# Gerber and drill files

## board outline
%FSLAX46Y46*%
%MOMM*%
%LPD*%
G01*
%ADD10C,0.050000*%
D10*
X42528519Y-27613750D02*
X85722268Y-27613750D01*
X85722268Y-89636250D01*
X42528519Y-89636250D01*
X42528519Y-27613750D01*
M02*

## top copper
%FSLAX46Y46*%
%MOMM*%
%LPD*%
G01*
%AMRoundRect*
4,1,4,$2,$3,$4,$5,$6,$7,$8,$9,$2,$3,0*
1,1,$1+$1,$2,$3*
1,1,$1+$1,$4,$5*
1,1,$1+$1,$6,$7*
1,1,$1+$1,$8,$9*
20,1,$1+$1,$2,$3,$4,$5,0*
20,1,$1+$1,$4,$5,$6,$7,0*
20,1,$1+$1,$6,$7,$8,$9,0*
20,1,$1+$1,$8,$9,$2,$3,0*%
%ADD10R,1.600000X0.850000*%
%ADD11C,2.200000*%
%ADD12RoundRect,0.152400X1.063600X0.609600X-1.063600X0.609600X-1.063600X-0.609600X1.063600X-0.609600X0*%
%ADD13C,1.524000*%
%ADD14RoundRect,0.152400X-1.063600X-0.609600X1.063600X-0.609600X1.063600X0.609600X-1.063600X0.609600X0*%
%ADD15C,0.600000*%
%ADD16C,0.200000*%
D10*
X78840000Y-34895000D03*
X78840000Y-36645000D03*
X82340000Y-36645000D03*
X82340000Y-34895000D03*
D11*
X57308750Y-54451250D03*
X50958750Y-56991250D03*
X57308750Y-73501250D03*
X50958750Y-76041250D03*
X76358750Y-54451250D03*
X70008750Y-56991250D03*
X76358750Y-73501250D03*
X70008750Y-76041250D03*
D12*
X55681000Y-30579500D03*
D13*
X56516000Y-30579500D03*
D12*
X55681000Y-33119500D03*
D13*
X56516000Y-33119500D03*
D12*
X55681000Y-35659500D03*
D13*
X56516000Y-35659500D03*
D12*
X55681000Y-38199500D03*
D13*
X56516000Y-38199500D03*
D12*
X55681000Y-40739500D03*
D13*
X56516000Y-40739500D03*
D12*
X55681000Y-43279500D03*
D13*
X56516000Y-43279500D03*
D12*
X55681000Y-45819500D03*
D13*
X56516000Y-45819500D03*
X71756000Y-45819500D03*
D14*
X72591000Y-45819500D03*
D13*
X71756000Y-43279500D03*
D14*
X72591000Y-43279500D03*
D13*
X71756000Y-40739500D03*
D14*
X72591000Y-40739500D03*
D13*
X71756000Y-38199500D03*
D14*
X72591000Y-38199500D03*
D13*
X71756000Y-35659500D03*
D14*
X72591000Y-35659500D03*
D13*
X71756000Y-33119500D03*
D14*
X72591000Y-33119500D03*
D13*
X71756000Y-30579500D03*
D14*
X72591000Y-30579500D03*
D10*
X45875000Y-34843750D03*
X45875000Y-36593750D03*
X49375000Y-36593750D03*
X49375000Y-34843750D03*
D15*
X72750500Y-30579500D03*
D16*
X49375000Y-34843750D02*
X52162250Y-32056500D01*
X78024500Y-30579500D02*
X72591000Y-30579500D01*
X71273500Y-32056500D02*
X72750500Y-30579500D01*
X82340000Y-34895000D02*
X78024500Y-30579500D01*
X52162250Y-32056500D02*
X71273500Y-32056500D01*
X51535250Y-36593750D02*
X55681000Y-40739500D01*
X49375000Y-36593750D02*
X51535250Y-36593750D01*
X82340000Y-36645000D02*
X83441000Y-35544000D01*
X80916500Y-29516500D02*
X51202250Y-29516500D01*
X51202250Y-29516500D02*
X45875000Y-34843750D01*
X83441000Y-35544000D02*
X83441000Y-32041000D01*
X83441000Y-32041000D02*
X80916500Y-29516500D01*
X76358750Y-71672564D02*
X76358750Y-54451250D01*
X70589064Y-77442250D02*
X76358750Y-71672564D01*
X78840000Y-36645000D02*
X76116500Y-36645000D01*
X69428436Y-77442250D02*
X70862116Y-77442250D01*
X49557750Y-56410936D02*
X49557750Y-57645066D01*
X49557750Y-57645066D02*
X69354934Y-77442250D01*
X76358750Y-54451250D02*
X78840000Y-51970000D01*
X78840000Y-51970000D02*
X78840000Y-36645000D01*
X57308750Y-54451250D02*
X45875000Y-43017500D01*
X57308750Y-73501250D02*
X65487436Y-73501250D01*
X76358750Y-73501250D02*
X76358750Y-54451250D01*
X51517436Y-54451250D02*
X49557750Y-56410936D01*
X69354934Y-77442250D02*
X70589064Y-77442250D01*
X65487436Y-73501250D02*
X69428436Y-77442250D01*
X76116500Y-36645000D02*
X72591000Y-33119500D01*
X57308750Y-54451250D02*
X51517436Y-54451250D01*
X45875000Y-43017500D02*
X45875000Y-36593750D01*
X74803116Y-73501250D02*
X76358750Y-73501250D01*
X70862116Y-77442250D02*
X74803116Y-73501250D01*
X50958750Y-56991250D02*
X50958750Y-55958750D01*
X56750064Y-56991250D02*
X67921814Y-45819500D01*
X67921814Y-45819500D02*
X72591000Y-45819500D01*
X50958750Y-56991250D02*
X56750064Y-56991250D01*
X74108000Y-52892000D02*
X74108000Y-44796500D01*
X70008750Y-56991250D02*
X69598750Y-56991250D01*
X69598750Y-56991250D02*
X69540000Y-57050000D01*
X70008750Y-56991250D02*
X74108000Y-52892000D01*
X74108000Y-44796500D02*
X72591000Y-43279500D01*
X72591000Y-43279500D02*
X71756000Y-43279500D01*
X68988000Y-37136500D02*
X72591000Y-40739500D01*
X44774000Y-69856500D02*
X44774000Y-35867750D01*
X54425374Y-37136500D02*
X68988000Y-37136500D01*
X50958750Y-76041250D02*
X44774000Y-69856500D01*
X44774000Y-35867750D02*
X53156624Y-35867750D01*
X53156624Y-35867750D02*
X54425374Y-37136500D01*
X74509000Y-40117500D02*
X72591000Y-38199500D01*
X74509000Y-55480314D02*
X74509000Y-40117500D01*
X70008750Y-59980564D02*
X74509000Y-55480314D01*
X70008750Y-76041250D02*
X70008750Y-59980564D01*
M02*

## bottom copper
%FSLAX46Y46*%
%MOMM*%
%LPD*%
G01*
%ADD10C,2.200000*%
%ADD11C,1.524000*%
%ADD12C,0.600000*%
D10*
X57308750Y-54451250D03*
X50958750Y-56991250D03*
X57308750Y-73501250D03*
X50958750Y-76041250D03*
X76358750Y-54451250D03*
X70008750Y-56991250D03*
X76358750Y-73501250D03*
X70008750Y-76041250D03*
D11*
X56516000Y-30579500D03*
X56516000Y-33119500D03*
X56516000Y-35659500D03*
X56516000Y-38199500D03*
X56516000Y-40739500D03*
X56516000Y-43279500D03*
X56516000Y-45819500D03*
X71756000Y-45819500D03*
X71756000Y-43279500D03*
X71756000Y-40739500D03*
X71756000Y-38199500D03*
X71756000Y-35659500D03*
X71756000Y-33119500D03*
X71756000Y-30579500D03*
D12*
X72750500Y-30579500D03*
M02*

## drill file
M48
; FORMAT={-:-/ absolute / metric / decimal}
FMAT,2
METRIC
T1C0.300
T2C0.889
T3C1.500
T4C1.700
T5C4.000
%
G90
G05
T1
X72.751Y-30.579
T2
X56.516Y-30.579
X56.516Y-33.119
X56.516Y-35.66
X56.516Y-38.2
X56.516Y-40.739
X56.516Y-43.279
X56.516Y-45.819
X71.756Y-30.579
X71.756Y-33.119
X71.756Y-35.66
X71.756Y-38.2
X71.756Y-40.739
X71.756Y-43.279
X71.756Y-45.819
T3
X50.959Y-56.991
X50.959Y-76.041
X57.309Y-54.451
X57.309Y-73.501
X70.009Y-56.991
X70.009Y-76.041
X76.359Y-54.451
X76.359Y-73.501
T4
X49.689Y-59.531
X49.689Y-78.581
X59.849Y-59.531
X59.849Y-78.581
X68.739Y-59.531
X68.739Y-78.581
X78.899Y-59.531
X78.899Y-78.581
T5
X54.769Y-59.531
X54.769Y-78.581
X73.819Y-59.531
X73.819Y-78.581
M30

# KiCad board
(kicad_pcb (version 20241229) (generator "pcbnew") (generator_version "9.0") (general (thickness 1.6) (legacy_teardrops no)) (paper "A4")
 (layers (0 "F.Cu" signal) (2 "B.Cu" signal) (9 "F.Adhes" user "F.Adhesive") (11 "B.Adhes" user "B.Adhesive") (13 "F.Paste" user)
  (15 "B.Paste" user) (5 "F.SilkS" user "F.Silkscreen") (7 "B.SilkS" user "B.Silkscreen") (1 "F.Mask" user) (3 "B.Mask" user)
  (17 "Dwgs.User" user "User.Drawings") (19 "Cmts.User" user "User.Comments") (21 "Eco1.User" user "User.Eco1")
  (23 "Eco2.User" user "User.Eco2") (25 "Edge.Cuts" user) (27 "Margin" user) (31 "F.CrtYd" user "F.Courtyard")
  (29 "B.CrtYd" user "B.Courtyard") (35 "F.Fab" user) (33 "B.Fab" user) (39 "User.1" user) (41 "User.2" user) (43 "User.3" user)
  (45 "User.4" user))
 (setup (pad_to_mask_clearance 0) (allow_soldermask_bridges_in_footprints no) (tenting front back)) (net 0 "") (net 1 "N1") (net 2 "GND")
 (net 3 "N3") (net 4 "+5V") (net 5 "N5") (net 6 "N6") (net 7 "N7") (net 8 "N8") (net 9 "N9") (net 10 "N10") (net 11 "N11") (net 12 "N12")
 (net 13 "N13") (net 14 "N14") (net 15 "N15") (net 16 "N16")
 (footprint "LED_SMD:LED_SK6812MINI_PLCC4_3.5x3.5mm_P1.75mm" (layer "F.Cu") (at 80.59 35.77)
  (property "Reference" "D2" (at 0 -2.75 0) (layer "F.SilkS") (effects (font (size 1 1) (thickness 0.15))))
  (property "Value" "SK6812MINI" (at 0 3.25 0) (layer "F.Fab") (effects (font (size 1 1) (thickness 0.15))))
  (pad "1" smd rect (at -1.75 -0.875) (size 1.6 0.85) (layers "F.Cu" "F.Mask" "F.Paste") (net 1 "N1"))
  (pad "2" smd rect (at -1.75 0.875) (size 1.6 0.85) (layers "F.Cu" "F.Mask" "F.Paste") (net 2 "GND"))
  (pad "3" smd rect (at 1.75 0.875) (size 1.6 0.85) (layers "F.Cu" "F.Mask" "F.Paste") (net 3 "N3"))
  (pad "4" smd rect (at 1.75 -0.875) (size 1.6 0.85) (layers "F.Cu" "F.Mask" "F.Paste") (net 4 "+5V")))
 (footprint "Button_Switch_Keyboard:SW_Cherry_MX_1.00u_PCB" (layer "F.Cu") (at 57.30875 54.45125)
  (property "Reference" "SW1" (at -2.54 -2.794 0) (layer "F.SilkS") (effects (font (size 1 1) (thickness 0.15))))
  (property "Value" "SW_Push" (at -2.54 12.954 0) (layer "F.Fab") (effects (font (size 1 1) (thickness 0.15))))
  (pad "" np_thru_hole circle (at -7.62 5.08) (size 1.7 1.7) (drill 1.7) (layers "*.Cu" "*.Mask"))
  (pad "" np_thru_hole circle (at -2.54 5.08) (size 4 4) (drill 4) (layers "*.Cu" "*.Mask"))
  (pad "" np_thru_hole circle (at 2.54 5.08) (size 1.7 1.7) (drill 1.7) (layers "*.Cu" "*.Mask"))
  (pad "1" thru_hole circle (at 0 0) (size 2.2 2.2) (drill 1.5) (layers "*.Cu" "*.Mask") (remove_unused_layers no) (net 2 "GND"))
  (pad "2" thru_hole circle (at -6.35 2.54) (size 2.2 2.2) (drill 1.5) (layers "*.Cu" "*.Mask") (remove_unused_layers no) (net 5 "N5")))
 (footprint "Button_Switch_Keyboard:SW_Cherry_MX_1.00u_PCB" (layer "F.Cu") (at 57.30875 73.50125)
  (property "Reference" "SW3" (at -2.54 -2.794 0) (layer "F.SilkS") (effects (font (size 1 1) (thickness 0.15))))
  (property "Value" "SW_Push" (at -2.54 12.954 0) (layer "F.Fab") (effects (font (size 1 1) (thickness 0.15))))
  (pad "" np_thru_hole circle (at -7.62 5.08) (size 1.7 1.7) (drill 1.7) (layers "*.Cu" "*.Mask"))
  (pad "" np_thru_hole circle (at -2.54 5.08) (size 4 4) (drill 4) (layers "*.Cu" "*.Mask"))
  (pad "" np_thru_hole circle (at 2.54 5.08) (size 1.7 1.7) (drill 1.7) (layers "*.Cu" "*.Mask"))
  (pad "1" thru_hole circle (at 0 0) (size 2.2 2.2) (drill 1.5) (layers "*.Cu" "*.Mask") (remove_unused_layers no) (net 2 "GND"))
  (pad "2" thru_hole circle (at -6.35 2.54) (size 2.2 2.2) (drill 1.5) (layers "*.Cu" "*.Mask") (remove_unused_layers no) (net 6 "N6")))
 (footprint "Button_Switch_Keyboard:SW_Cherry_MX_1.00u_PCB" (layer "F.Cu") (at 76.35875 54.45125)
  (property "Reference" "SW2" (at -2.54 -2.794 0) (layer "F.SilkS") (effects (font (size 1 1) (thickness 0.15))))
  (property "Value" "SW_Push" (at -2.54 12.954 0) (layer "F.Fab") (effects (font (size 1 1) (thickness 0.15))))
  (pad "" np_thru_hole circle (at -7.62 5.08) (size 1.7 1.7) (drill 1.7) (layers "*.Cu" "*.Mask"))
  (pad "" np_thru_hole circle (at -2.54 5.08) (size 4 4) (drill 4) (layers "*.Cu" "*.Mask"))
  (pad "" np_thru_hole circle (at 2.54 5.08) (size 1.7 1.7) (drill 1.7) (layers "*.Cu" "*.Mask"))
  (pad "1" thru_hole circle (at 0 0) (size 2.2 2.2) (drill 1.5) (layers "*.Cu" "*.Mask") (remove_unused_layers no) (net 2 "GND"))
  (pad "2" thru_hole circle (at -6.35 2.54) (size 2.2 2.2) (drill 1.5) (layers "*.Cu" "*.Mask") (remove_unused_layers no) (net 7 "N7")))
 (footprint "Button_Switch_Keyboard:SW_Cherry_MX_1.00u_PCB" (layer "F.Cu") (at 76.35875 73.50125)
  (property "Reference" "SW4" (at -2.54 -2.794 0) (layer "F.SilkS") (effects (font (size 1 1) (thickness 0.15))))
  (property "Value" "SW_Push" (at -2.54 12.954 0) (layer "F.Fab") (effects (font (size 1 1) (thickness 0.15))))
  (pad "" np_thru_hole circle (at -7.62 5.08) (size 1.7 1.7) (drill 1.7) (layers "*.Cu" "*.Mask"))
  (pad "" np_thru_hole circle (at -2.54 5.08) (size 4 4) (drill 4) (layers "*.Cu" "*.Mask"))
  (pad "" np_thru_hole circle (at 2.54 5.08) (size 1.7 1.7) (drill 1.7) (layers "*.Cu" "*.Mask"))
  (pad "1" thru_hole circle (at 0 0) (size 2.2 2.2) (drill 1.5) (layers "*.Cu" "*.Mask") (remove_unused_layers no) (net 2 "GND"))
  (pad "2" thru_hole circle (at -6.35 2.54) (size 2.2 2.2) (drill 1.5) (layers "*.Cu" "*.Mask") (remove_unused_layers no) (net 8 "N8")))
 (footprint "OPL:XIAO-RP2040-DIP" (layer "F.Cu") (at 64.136 38.1995)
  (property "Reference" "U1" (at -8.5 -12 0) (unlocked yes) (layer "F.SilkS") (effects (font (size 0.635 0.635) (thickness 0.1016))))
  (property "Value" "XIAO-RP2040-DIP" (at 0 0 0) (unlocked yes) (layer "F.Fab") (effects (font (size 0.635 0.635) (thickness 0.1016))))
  (pad "1" smd roundrect (at -8.455 -7.62 180) (size 2.432 1.524) (layers "F.Cu" "F.Mask") (roundrect_rratio 0.1) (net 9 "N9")
   (thermal_bridge_angle 45))
  (pad "1" thru_hole circle (at -7.62 -7.62 180) (size 1.524 1.524) (drill 0.889) (layers "*.Cu" "*.Mask") (remove_unused_layers no)
   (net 9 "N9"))
  (pad "2" smd roundrect (at -8.455 -5.08 180) (size 2.432 1.524) (layers "F.Cu" "F.Mask") (roundrect_rratio 0.1) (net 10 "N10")
   (thermal_bridge_angle 45))
  (pad "2" thru_hole circle (at -7.62 -5.08 180) (size 1.524 1.524) (drill 0.889) (layers "*.Cu" "*.Mask") (remove_unused_layers no)
   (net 10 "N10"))
  (pad "3" smd roundrect (at -8.455 -2.54 180) (size 2.432 1.524) (layers "F.Cu" "F.Mask") (roundrect_rratio 0.1) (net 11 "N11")
   (thermal_bridge_angle 45))
  (pad "3" thru_hole circle (at -7.62 -2.54 180) (size 1.524 1.524) (drill 0.889) (layers "*.Cu" "*.Mask") (remove_unused_layers no)
   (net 11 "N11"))
  (pad "4" smd roundrect (at -8.455 0 180) (size 2.432 1.524) (layers "F.Cu" "F.Mask") (roundrect_rratio 0.1) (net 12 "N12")
   (thermal_bridge_angle 45))
  (pad "4" thru_hole circle (at -7.62 0 180) (size 1.524 1.524) (drill 0.889) (layers "*.Cu" "*.Mask") (remove_unused_layers no)
   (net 12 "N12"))
  (pad "5" smd roundrect (at -8.455 2.54 180) (size 2.432 1.524) (layers "F.Cu" "F.Mask") (roundrect_rratio 0.1) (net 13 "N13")
   (thermal_bridge_angle 45))
  (pad "5" thru_hole circle (at -7.62 2.54 180) (size 1.524 1.524) (drill 0.889) (layers "*.Cu" "*.Mask") (remove_unused_layers no)
   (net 13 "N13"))
  (pad "6" smd roundrect (at -8.455 5.08 180) (size 2.432 1.524) (layers "F.Cu" "F.Mask") (roundrect_rratio 0.1) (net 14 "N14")
   (thermal_bridge_angle 45))
  (pad "6" thru_hole circle (at -7.62 5.08 180) (size 1.524 1.524) (drill 0.889) (layers "*.Cu" "*.Mask") (remove_unused_layers no)
   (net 14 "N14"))
  (pad "7" smd roundrect (at -8.455 7.62 180) (size 2.432 1.524) (layers "F.Cu" "F.Mask") (roundrect_rratio 0.1) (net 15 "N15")
   (thermal_bridge_angle 45))
  (pad "7" thru_hole circle (at -7.62 7.62 180) (size 1.524 1.524) (drill 0.889) (layers "*.Cu" "*.Mask") (remove_unused_layers no)
   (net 15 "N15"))
  (pad "8" thru_hole circle (at 7.62 7.62) (size 1.524 1.524) (drill 0.889) (layers "*.Cu" "*.Mask") (remove_unused_layers no) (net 5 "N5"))
  (pad "8" smd roundrect (at 8.455 7.62) (size 2.432 1.524) (layers "F.Cu" "F.Mask") (roundrect_rratio 0.1) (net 5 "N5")
   (thermal_bridge_angle 45))
  (pad "9" thru_hole circle (at 7.62 5.08) (size 1.524 1.524) (drill 0.889) (layers "*.Cu" "*.Mask") (remove_unused_layers no) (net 7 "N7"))
  (pad "9" smd roundrect (at 8.455 5.08) (size 2.432 1.524) (layers "F.Cu" "F.Mask") (roundrect_rratio 0.1) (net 7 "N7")
   (thermal_bridge_angle 45))
  (pad "10" thru_hole circle (at 7.62 2.54) (size 1.524 1.524) (drill 0.889) (layers "*.Cu" "*.Mask") (remove_unused_layers no) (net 6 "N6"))
  (pad "10" smd roundrect (at 8.455 2.54) (size 2.432 1.524) (layers "F.Cu" "F.Mask") (roundrect_rratio 0.1) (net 6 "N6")
   (thermal_bridge_angle 45))
  (pad "11" thru_hole circle (at 7.62 0) (size 1.524 1.524) (drill 0.889) (layers "*.Cu" "*.Mask") (remove_unused_layers no) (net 8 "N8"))
  (pad "11" smd roundrect (at 8.455 0) (size 2.432 1.524) (layers "F.Cu" "F.Mask") (roundrect_rratio 0.1) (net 8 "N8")
   (thermal_bridge_angle 45))
  (pad "12" thru_hole circle (at 7.62 -2.54) (size 1.524 1.524) (drill 0.889) (layers "*.Cu" "*.Mask") (remove_unused_layers no)
   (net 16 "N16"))
  (pad "12" smd roundrect (at 8.455 -2.54) (size 2.432 1.524) (layers "F.Cu" "F.Mask") (roundrect_rratio 0.1) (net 16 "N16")
   (thermal_bridge_angle 45))
  (pad "13" thru_hole circle (at 7.62 -5.08) (size 1.524 1.524) (drill 0.889) (layers "*.Cu" "*.Mask") (remove_unused_layers no)
   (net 2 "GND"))
  (pad "13" smd roundrect (at 8.455 -5.08) (size 2.432 1.524) (layers "F.Cu" "F.Mask") (roundrect_rratio 0.1) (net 2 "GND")
   (thermal_bridge_angle 45))
  (pad "14" thru_hole circle (at 7.62 -7.62) (size 1.524 1.524) (drill 0.889) (layers "*.Cu" "*.Mask") (remove_unused_layers no)
   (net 4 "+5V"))
  (pad "14" smd roundrect (at 8.455 -7.62) (size 2.432 1.524) (layers "F.Cu" "F.Mask") (roundrect_rratio 0.1) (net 4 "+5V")
   (thermal_bridge_angle 45)))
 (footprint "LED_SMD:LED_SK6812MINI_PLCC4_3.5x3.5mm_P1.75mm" (layer "F.Cu") (at 47.625 35.71875)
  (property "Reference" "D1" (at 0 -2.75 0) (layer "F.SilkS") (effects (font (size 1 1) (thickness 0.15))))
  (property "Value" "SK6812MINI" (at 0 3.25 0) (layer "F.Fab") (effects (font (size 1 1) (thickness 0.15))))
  (pad "1" smd rect (at -1.75 -0.875) (size 1.6 0.85) (layers "F.Cu" "F.Mask" "F.Paste") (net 3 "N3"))
  (pad "2" smd rect (at -1.75 0.875) (size 1.6 0.85) (layers "F.Cu" "F.Mask" "F.Paste") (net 2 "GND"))
  (pad "3" smd rect (at 1.75 0.875) (size 1.6 0.85) (layers "F.Cu" "F.Mask" "F.Paste") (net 13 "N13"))
  (pad "4" smd rect (at 1.75 -0.875) (size 1.6 0.85) (layers "F.Cu" "F.Mask" "F.Paste") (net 4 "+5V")))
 (gr_rect (start 42.528519 27.61375) (end 85.722268 89.63625) (stroke (width 0.05) (type default)) (fill no) (layer "Edge.Cuts"))
 (segment (start 49.375 34.84375) (end 52.16225 32.0565) (width 0.2) (layer "F.Cu") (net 4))
 (segment (start 78.0245 30.5795) (end 72.591 30.5795) (width 0.2) (layer "F.Cu") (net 4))
 (segment (start 71.2735 32.0565) (end 72.7505 30.5795) (width 0.2) (layer "F.Cu") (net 4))
 (segment (start 82.34 34.895) (end 78.0245 30.5795) (width 0.2) (layer "F.Cu") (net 4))
 (segment (start 52.16225 32.0565) (end 71.2735 32.0565) (width 0.2) (layer "F.Cu") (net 4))
 (via (at 72.7505 30.5795) (size 0.6) (drill 0.3) (layers "F.Cu" "B.Cu") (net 4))
 (segment (start 51.53525 36.59375) (end 55.681 40.7395) (width 0.2) (layer "F.Cu") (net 13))
 (segment (start 49.375 36.59375) (end 51.53525 36.59375) (width 0.2) (layer "F.Cu") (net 13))
 (segment (start 82.34 36.645) (end 83.441 35.544) (width 0.2) (layer "F.Cu") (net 3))
 (segment (start 80.9165 29.5165) (end 51.20225 29.5165) (width 0.2) (layer "F.Cu") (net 3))
 (segment (start 51.20225 29.5165) (end 45.875 34.84375) (width 0.2) (layer "F.Cu") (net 3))
 (segment (start 83.441 35.544) (end 83.441 32.041) (width 0.2) (layer "F.Cu") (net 3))
 (segment (start 83.441 32.041) (end 80.9165 29.5165) (width 0.2) (layer "F.Cu") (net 3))
 (segment (start 76.35875 71.672564) (end 76.35875 54.45125) (width 0.2) (layer "F.Cu") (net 2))
 (segment (start 70.589064 77.44225) (end 76.35875 71.672564) (width 0.2) (layer "F.Cu") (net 2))
 (segment (start 78.84 36.645) (end 76.1165 36.645) (width 0.2) (layer "F.Cu") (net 2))
 (segment (start 69.428436 77.44225) (end 70.862116 77.44225) (width 0.2) (layer "F.Cu") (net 2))
 (segment (start 49.55775 56.410936) (end 49.55775 57.645066) (width 0.2) (layer "F.Cu") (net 2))
 (segment (start 49.55775 57.645066) (end 69.354934 77.44225) (width 0.2) (layer "F.Cu") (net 2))
 (segment (start 76.35875 54.45125) (end 78.84 51.97) (width 0.2) (layer "F.Cu") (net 2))
 (segment (start 78.84 51.97) (end 78.84 36.645) (width 0.2) (layer "F.Cu") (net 2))
 (segment (start 57.30875 54.45125) (end 45.875 43.0175) (width 0.2) (layer "F.Cu") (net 2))
 (segment (start 57.30875 73.50125) (end 65.487436 73.50125) (width 0.2) (layer "F.Cu") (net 2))
 (segment (start 76.35875 73.50125) (end 76.35875 54.45125) (width 0.2) (layer "F.Cu") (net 2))
 (segment (start 51.517436 54.45125) (end 49.55775 56.410936) (width 0.2) (layer "F.Cu") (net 2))
 (segment (start 69.354934 77.44225) (end 70.589064 77.44225) (width 0.2) (layer "F.Cu") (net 2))
 (segment (start 65.487436 73.50125) (end 69.428436 77.44225) (width 0.2) (layer "F.Cu") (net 2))
 (segment (start 76.1165 36.645) (end 72.591 33.1195) (width 0.2) (layer "F.Cu") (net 2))
 (segment (start 57.30875 54.45125) (end 51.517436 54.45125) (width 0.2) (layer "F.Cu") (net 2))
 (segment (start 45.875 43.0175) (end 45.875 36.59375) (width 0.2) (layer "F.Cu") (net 2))
 (segment (start 74.803116 73.50125) (end 76.35875 73.50125) (width 0.2) (layer "F.Cu") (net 2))
 (segment (start 70.862116 77.44225) (end 74.803116 73.50125) (width 0.2) (layer "F.Cu") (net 2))
 (segment (start 50.95875 56.99125) (end 50.95875 55.95875) (width 0.2) (layer "F.Cu") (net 5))
 (segment (start 56.750064 56.99125) (end 67.921814 45.8195) (width 0.2) (layer "F.Cu") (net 5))
 (segment (start 67.921814 45.8195) (end 72.591 45.8195) (width 0.2) (layer "F.Cu") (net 5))
 (segment (start 50.95875 56.99125) (end 56.750064 56.99125) (width 0.2) (layer "F.Cu") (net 5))
 (segment (start 74.108 52.892) (end 74.108 44.7965) (width 0.2) (layer "F.Cu") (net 7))
 (segment (start 70.00875 56.99125) (end 69.59875 56.99125) (width 0.2) (layer "F.Cu") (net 7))
 (segment (start 69.59875 56.99125) (end 69.54 57.05) (width 0.2) (layer "F.Cu") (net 7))
 (segment (start 70.00875 56.99125) (end 74.108 52.892) (width 0.2) (layer "F.Cu") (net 7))
 (segment (start 74.108 44.7965) (end 72.591 43.2795) (width 0.2) (layer "F.Cu") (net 7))
 (segment (start 72.591 43.2795) (end 71.756 43.2795) (width 0.2) (layer "F.Cu") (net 7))
 (segment (start 68.988 37.1365) (end 72.591 40.7395) (width 0.2) (layer "F.Cu") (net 6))
 (segment (start 44.774 69.8565) (end 44.774 35.86775) (width 0.2) (layer "F.Cu") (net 6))
 (segment (start 54.425374 37.1365) (end 68.988 37.1365) (width 0.2) (layer "F.Cu") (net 6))
 (segment (start 50.95875 76.04125) (end 44.774 69.8565) (width 0.2) (layer "F.Cu") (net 6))
 (segment (start 44.774 35.86775) (end 53.156624 35.86775) (width 0.2) (layer "F.Cu") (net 6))
 (segment (start 53.156624 35.86775) (end 54.425374 37.1365) (width 0.2) (layer "F.Cu") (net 6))
 (segment (start 74.509 40.1175) (end 72.591 38.1995) (width 0.2) (layer "F.Cu") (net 8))
 (segment (start 74.509 55.480314) (end 74.509 40.1175) (width 0.2) (layer "F.Cu") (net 8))
 (segment (start 70.00875 59.980564) (end 74.509 55.480314) (width 0.2) (layer "F.Cu") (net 8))
 (segment (start 70.00875 76.04125) (end 70.00875 59.980564) (width 0.2) (layer "F.Cu") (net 8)))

